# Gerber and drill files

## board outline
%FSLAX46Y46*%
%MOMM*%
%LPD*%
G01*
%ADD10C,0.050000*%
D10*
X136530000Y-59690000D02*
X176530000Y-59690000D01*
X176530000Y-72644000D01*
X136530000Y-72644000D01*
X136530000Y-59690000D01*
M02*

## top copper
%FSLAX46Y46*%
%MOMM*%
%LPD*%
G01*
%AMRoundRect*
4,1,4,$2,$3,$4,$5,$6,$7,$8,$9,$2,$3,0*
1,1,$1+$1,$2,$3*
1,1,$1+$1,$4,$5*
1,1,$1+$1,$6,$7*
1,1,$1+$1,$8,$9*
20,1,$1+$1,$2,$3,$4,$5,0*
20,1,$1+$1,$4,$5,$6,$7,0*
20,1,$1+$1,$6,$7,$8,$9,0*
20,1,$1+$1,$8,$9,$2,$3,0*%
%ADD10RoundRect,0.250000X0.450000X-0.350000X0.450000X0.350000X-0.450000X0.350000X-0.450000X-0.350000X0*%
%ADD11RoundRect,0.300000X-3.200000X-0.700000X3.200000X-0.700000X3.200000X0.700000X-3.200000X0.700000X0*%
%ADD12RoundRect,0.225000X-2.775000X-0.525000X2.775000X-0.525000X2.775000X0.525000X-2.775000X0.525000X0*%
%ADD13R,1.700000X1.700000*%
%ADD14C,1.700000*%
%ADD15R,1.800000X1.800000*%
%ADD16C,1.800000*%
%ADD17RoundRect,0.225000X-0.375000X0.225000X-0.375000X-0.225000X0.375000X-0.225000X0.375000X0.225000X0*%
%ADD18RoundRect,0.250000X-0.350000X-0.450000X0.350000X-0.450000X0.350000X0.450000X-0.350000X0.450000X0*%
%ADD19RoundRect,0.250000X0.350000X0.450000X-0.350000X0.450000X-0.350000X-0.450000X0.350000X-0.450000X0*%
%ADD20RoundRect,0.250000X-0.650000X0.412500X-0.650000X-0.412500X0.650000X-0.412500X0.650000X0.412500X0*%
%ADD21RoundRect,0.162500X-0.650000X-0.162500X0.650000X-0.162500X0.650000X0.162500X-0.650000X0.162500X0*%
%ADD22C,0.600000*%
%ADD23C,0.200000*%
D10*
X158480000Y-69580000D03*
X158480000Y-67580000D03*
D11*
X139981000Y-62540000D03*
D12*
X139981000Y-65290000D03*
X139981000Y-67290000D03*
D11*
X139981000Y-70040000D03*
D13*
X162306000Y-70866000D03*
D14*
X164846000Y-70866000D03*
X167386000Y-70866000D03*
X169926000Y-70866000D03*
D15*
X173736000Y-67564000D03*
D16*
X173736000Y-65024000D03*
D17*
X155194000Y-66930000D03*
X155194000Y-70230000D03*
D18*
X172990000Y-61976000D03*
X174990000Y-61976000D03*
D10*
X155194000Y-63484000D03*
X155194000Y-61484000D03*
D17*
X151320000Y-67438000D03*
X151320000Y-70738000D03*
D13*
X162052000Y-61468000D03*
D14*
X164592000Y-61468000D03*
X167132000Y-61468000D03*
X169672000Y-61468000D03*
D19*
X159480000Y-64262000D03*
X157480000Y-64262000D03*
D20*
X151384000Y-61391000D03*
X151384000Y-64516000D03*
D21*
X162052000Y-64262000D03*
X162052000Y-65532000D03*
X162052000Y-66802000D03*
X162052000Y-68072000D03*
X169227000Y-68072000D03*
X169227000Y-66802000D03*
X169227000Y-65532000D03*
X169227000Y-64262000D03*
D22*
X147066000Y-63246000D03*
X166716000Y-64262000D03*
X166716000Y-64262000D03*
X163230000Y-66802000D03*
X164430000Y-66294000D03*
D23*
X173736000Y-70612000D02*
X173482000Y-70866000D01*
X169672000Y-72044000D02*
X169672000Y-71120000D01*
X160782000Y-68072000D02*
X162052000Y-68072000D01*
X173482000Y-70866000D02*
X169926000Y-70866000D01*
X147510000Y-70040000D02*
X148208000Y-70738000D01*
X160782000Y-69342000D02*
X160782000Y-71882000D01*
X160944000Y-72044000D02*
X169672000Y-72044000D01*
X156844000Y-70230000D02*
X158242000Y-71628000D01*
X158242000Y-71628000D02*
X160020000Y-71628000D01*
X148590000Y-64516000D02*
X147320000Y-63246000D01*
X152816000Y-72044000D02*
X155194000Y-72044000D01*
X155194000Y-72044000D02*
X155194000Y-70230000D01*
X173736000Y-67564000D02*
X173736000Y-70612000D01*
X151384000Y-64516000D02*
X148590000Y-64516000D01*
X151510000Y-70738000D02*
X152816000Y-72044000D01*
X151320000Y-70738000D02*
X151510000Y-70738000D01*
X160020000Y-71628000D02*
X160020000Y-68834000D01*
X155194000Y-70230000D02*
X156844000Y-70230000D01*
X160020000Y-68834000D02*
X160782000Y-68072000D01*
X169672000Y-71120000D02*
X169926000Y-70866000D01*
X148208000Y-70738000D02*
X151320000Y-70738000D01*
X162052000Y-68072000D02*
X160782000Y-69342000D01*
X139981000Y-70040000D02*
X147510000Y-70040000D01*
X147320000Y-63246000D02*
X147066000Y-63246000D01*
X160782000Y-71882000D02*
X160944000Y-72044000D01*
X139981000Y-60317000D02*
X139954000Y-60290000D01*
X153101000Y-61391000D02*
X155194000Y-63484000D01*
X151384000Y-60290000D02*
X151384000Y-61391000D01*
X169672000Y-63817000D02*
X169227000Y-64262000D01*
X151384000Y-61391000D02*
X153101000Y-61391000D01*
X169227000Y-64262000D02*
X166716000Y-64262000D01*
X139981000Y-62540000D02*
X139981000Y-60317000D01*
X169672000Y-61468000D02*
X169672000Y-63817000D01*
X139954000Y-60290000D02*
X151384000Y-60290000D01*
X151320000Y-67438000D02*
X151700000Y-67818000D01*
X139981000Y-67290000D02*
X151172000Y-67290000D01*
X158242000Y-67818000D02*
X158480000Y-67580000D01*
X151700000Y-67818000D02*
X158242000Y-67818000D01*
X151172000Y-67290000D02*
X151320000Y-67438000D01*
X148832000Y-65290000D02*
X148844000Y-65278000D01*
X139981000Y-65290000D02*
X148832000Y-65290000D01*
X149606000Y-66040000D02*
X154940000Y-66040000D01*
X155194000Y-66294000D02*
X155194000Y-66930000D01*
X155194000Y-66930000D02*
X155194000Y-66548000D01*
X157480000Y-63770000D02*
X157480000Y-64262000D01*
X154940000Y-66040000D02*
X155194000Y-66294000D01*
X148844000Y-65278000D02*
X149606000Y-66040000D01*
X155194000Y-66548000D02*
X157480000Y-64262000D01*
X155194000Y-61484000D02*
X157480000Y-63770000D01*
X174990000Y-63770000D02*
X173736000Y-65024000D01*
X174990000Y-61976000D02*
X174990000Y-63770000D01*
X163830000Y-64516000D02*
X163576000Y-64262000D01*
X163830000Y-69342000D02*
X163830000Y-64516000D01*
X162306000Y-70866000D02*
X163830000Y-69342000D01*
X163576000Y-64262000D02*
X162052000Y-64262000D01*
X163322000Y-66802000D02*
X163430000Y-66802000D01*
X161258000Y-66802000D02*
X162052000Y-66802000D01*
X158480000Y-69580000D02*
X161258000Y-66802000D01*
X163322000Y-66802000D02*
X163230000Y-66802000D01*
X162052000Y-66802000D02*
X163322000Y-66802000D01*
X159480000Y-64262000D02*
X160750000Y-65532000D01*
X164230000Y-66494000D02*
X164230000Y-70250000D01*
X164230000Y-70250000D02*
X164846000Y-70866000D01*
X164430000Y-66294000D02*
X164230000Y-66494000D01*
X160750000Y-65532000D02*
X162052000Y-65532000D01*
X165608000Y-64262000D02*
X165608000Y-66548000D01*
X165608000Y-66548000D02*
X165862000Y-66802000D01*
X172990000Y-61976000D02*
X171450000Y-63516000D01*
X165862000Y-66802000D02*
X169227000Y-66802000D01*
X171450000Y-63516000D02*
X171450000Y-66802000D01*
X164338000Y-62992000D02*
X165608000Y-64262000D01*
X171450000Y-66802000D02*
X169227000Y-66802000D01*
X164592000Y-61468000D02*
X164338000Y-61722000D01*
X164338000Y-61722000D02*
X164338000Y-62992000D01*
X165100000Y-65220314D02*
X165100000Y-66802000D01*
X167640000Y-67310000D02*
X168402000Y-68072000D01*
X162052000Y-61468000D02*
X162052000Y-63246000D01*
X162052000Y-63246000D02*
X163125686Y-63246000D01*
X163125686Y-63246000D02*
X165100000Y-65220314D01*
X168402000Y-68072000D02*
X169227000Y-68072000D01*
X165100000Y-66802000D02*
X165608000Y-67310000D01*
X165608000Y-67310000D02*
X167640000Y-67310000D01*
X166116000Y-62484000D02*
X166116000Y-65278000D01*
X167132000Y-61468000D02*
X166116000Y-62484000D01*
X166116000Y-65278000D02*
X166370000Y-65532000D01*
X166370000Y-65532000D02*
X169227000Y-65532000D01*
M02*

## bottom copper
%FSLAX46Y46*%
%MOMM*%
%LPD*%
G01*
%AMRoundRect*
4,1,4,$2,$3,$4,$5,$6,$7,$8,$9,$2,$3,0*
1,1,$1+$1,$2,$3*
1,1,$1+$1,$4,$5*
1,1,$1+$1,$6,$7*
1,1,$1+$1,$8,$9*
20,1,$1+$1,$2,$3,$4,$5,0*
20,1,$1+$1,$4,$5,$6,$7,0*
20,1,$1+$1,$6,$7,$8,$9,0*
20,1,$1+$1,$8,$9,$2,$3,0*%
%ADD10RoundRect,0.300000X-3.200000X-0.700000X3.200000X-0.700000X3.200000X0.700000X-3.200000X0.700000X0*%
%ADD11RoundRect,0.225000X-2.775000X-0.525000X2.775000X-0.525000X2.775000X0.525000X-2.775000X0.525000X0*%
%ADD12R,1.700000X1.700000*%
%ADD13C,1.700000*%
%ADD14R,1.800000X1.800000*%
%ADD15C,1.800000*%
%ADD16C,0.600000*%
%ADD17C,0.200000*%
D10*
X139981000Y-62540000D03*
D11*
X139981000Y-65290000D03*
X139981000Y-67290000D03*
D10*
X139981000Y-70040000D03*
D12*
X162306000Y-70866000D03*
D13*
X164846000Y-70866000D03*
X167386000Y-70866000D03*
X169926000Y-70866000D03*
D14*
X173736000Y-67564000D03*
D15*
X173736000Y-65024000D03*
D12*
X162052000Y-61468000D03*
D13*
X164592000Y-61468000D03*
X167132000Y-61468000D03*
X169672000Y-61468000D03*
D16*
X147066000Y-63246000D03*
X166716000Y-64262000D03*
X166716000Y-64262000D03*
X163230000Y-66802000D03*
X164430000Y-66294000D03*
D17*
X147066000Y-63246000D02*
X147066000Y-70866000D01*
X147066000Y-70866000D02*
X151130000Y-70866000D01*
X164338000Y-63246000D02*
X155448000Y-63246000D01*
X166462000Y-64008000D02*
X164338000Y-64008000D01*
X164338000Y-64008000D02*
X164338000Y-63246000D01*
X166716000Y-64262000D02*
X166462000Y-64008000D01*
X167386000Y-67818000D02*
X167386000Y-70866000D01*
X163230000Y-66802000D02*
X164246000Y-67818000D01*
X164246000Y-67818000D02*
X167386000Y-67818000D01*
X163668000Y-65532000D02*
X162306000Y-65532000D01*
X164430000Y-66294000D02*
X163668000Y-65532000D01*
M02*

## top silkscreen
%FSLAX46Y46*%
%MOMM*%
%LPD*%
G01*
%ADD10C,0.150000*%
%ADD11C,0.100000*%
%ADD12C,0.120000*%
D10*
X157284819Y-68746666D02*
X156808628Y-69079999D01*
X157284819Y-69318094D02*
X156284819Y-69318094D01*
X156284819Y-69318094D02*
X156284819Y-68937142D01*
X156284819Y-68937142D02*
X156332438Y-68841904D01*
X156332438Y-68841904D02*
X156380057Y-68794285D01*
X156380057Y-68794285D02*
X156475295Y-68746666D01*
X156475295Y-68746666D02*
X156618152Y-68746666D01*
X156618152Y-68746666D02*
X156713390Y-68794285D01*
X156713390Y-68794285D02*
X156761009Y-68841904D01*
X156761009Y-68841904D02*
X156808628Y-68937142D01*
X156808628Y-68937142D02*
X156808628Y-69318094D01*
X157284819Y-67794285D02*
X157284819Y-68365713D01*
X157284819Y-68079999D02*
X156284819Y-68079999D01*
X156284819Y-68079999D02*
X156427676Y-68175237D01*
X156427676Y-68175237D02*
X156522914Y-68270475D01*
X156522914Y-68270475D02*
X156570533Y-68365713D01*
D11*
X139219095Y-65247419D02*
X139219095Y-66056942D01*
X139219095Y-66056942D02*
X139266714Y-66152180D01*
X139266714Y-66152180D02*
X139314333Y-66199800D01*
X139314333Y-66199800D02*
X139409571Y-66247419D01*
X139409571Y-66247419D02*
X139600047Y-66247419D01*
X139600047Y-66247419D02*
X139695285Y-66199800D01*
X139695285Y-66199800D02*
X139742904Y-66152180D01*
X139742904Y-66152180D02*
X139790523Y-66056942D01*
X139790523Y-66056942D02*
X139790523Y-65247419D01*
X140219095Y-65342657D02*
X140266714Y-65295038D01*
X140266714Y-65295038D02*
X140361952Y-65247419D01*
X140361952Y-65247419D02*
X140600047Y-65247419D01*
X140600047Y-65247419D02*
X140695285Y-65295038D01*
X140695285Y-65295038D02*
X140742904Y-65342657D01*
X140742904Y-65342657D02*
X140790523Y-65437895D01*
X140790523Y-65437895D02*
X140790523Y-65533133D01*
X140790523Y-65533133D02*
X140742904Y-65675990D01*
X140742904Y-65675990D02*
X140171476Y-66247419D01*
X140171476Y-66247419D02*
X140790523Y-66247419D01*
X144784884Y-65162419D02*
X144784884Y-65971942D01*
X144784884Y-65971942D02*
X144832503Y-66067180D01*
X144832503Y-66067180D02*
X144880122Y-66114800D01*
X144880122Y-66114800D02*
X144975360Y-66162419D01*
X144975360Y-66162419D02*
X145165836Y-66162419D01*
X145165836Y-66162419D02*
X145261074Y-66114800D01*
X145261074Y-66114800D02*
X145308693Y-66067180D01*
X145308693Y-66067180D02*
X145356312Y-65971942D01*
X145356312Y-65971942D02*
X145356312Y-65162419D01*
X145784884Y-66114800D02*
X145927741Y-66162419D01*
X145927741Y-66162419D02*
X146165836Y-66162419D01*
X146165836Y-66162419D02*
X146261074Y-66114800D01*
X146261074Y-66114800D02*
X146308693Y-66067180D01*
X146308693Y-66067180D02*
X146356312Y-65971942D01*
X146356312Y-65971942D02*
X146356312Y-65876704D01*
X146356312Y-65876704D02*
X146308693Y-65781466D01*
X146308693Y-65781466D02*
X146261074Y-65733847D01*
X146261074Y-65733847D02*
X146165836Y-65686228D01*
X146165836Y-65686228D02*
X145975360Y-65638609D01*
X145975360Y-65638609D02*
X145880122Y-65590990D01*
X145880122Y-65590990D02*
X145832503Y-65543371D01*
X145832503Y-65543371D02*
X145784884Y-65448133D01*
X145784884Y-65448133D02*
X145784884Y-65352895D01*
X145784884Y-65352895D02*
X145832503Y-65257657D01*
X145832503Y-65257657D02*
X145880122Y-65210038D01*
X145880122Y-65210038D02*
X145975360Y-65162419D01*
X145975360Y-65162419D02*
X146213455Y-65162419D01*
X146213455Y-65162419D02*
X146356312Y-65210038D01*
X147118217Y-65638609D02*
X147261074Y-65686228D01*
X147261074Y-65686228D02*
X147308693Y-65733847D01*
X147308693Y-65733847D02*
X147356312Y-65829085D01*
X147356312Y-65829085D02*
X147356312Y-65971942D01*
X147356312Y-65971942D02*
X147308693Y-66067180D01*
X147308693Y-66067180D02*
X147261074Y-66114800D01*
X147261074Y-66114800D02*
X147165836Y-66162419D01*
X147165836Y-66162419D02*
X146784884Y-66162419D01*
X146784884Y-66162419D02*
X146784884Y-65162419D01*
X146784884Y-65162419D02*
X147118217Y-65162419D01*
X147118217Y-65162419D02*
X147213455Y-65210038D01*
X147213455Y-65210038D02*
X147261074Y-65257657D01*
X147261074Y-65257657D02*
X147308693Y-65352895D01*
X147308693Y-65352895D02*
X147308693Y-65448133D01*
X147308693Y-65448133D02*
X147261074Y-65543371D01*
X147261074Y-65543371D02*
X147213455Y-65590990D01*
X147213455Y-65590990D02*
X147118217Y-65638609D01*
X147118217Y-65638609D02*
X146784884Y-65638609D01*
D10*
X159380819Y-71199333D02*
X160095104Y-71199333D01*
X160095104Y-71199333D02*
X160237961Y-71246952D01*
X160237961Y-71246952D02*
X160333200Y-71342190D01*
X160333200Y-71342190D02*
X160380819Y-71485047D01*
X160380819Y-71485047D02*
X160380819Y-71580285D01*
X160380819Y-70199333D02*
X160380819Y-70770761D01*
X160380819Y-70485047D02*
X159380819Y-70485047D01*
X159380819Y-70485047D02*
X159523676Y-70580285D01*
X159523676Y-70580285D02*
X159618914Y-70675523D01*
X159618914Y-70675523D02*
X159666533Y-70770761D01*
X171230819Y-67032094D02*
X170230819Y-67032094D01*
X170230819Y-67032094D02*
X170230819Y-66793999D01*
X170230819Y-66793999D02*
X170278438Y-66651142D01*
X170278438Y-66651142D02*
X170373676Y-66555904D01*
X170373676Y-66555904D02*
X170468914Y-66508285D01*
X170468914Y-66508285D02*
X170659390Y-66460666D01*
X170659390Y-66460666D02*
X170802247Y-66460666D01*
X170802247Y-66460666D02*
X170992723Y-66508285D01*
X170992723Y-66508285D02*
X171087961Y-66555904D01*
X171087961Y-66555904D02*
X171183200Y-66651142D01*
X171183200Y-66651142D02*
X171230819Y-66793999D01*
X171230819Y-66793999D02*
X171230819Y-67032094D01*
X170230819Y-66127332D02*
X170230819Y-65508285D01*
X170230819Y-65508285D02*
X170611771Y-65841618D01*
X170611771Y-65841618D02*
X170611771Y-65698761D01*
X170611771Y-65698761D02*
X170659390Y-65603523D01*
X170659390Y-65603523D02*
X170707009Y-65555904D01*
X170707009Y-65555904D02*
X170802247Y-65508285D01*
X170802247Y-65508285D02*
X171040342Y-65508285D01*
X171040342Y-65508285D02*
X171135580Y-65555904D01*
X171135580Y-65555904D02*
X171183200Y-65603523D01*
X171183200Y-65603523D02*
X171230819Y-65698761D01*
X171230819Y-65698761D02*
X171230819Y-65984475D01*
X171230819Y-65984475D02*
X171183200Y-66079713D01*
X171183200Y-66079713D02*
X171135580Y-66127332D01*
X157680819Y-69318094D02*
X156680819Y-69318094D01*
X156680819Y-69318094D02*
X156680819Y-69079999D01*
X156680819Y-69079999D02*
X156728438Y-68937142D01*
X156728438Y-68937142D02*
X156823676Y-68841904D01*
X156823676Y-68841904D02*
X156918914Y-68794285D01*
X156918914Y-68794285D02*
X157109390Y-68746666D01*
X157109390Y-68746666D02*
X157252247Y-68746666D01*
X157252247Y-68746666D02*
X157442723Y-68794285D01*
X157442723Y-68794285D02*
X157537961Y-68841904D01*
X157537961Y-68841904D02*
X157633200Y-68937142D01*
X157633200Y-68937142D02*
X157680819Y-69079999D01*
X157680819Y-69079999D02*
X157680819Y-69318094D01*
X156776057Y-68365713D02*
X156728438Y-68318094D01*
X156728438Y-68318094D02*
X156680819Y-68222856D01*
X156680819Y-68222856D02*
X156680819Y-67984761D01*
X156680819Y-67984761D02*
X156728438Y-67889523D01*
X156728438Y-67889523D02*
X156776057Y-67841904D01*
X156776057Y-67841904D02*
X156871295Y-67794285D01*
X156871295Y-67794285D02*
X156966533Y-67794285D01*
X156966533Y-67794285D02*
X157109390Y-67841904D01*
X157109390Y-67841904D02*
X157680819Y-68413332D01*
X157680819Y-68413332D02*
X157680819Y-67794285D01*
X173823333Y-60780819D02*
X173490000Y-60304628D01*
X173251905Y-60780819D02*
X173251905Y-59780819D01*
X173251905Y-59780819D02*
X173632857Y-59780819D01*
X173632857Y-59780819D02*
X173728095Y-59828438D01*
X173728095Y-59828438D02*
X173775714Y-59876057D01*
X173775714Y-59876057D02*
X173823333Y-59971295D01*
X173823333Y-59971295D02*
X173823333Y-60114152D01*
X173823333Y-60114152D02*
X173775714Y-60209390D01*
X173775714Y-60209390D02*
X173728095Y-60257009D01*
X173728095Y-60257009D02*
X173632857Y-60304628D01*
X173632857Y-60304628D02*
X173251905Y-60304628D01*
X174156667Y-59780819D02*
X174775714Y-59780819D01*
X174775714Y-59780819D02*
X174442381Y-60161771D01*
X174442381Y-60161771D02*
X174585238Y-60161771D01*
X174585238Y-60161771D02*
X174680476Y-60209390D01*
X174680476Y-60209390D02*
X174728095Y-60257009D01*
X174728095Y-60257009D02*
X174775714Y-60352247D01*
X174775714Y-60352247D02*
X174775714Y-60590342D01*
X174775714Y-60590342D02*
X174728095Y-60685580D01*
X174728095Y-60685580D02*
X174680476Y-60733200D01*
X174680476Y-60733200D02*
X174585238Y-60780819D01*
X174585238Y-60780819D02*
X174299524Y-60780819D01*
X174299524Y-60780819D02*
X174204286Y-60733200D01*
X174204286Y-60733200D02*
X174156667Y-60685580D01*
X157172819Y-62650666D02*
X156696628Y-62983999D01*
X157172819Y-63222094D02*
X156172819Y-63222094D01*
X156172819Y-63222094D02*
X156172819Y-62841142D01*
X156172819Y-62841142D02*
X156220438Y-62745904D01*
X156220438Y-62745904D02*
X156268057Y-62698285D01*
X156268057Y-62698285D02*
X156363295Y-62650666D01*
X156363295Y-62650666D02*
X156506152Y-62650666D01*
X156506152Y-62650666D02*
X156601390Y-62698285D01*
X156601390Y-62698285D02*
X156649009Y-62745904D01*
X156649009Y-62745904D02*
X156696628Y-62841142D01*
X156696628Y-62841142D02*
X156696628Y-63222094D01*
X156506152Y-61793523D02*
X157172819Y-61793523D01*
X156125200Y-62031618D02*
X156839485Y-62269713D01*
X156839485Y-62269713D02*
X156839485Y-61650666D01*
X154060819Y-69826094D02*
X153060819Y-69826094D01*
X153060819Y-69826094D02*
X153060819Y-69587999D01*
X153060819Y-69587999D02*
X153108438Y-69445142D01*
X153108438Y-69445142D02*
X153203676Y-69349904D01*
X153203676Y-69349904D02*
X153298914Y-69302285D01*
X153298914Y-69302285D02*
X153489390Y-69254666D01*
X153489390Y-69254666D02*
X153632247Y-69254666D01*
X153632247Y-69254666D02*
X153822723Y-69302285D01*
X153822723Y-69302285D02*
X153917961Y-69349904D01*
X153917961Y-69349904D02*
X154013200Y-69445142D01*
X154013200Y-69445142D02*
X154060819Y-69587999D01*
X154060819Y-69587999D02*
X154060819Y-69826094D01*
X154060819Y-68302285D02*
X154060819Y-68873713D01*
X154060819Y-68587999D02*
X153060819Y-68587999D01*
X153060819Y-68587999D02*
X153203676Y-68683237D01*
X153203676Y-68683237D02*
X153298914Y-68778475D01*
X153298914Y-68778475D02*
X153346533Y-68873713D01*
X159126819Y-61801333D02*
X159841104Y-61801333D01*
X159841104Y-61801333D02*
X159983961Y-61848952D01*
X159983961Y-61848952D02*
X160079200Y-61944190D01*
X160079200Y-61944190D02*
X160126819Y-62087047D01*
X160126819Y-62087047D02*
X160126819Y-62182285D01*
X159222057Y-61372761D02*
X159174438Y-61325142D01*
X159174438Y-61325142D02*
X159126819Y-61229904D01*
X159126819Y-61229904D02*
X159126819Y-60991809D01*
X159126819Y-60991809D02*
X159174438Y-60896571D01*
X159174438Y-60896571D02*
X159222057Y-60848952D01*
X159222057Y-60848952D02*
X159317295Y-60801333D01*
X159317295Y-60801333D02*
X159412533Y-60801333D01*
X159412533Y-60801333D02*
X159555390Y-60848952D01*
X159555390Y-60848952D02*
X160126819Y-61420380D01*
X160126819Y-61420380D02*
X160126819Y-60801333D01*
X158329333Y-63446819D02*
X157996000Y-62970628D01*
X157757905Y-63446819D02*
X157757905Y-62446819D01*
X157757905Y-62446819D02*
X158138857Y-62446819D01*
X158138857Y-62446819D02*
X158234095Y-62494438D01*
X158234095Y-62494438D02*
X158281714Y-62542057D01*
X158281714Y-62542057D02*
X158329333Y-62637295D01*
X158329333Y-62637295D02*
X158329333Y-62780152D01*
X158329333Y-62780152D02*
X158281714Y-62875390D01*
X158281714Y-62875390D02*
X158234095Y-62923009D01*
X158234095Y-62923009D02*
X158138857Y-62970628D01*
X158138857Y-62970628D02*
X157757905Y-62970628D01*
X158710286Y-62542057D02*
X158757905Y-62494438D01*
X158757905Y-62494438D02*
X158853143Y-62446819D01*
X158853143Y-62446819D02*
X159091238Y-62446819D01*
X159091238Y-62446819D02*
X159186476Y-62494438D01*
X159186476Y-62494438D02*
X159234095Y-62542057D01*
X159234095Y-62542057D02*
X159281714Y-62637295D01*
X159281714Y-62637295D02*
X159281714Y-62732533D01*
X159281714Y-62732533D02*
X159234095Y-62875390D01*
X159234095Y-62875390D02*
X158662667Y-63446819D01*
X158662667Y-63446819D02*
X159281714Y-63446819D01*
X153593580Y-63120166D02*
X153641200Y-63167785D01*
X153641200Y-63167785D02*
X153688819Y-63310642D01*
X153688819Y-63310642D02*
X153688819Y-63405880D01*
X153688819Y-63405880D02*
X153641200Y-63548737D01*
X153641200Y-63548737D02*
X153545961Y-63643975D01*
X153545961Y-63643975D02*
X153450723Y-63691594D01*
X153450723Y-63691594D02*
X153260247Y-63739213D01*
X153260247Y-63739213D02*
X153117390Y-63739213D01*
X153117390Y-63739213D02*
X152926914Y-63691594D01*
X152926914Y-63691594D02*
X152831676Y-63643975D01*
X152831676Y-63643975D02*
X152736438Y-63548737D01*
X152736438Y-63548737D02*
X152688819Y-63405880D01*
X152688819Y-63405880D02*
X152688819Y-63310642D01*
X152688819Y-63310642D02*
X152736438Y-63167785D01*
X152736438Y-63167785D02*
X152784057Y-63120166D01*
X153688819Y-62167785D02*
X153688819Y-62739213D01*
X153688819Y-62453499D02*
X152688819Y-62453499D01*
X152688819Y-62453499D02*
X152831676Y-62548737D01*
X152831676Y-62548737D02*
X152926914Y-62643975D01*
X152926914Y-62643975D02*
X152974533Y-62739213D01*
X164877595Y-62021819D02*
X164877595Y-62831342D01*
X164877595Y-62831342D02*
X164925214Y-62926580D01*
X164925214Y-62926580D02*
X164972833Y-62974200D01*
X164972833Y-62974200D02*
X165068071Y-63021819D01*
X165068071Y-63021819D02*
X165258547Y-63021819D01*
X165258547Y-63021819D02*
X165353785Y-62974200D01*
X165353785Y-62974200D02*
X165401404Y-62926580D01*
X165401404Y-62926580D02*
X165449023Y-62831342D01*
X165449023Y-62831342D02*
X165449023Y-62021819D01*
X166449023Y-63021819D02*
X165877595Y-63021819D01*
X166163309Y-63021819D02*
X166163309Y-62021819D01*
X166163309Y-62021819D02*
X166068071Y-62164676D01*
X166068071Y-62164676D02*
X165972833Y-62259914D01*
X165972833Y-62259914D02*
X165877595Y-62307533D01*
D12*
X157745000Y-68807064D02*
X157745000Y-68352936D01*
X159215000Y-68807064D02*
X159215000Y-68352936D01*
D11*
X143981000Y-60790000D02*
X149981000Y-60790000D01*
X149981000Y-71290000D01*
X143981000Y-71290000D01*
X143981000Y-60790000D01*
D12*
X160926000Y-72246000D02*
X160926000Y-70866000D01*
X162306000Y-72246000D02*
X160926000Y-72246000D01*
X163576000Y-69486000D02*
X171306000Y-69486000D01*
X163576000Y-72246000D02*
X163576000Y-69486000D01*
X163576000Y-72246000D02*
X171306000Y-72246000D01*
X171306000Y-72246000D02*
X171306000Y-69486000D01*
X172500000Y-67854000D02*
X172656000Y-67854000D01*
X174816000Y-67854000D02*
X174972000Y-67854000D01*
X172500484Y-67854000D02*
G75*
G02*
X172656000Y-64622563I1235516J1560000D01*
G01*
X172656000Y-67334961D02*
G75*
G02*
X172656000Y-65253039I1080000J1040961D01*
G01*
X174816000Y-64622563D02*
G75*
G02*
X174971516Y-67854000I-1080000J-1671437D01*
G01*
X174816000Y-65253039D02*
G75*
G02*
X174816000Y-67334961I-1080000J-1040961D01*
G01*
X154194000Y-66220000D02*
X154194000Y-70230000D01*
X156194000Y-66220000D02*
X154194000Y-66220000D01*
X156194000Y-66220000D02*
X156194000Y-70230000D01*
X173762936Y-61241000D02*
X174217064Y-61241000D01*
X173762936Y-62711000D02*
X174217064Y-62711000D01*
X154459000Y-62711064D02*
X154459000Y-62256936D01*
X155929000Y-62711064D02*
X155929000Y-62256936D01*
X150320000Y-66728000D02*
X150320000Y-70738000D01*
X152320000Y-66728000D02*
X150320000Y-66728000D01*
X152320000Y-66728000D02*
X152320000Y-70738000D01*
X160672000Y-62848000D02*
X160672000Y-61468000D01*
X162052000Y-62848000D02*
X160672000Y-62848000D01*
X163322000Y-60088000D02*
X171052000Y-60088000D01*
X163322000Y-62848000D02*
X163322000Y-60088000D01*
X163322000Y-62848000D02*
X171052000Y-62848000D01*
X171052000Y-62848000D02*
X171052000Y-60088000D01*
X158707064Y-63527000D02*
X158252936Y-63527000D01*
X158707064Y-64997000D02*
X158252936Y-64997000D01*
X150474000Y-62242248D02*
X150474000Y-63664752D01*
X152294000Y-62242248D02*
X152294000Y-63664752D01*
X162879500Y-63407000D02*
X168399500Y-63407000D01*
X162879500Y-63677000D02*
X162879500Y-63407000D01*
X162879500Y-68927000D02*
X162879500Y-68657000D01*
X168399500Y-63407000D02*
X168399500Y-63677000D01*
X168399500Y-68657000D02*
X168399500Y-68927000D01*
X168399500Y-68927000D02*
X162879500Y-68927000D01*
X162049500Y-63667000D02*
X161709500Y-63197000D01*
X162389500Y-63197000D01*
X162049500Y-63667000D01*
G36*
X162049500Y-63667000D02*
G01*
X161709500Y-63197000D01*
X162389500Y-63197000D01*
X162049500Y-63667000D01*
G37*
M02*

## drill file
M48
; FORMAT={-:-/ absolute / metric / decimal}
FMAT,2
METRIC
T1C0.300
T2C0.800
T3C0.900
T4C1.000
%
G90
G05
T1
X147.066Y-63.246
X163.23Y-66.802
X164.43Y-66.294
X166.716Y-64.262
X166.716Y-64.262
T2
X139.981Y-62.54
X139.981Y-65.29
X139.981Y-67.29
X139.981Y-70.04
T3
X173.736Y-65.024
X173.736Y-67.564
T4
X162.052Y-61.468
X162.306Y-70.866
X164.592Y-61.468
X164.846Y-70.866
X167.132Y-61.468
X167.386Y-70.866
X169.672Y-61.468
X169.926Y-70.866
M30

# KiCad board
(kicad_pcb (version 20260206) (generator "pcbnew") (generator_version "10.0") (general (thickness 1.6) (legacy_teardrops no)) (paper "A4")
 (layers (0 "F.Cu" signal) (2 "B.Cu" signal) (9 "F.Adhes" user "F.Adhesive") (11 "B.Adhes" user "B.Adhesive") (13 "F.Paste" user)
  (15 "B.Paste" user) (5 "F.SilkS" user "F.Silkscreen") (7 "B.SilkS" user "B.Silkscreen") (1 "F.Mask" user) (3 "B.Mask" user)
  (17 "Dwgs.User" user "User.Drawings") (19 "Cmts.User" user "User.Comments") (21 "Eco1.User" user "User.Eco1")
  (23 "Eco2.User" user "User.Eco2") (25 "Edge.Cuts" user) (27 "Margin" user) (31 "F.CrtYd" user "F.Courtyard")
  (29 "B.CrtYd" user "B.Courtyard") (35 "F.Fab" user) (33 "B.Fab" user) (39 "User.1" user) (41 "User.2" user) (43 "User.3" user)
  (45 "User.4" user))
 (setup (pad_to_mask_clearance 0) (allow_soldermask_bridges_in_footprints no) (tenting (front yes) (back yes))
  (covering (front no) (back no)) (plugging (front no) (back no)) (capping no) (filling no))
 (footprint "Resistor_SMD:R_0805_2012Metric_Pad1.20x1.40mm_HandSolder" (layer "F.Cu") (at 158.48 68.58 90)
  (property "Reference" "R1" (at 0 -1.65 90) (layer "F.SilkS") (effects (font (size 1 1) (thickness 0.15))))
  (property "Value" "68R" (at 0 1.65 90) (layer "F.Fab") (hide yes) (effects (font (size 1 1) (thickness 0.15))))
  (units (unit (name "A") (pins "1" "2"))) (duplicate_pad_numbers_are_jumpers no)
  (fp_line (start -0.227064 -0.735) (end 0.227064 -0.735) (stroke (width 0.12) (type solid)) (layer "F.SilkS"))
  (fp_line (start -0.227064 0.735) (end 0.227064 0.735) (stroke (width 0.12) (type solid)) (layer "F.SilkS"))
  (pad "1" smd roundrect (at -1 0 90) (size 1.2 1.4) (layers "F.Cu" "F.Mask" "F.Paste") (roundrect_rratio 0.208333) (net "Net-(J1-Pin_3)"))
  (pad "2" smd roundrect (at 1 0 90) (size 1.2 1.4) (layers "F.Cu" "F.Mask" "F.Paste") (roundrect_rratio 0.208333) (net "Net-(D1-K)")))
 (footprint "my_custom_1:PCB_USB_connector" (layer "F.Cu") (at 139.981 66.29)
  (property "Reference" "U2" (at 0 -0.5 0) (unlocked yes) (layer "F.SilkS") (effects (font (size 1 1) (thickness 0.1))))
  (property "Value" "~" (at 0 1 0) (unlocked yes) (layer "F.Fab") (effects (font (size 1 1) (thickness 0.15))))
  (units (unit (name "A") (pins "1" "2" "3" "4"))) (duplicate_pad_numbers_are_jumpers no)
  (fp_rect (start 4 -5.5) (end 10 5) (stroke (width 0.1) (type default)) (fill no) (layer "F.SilkS"))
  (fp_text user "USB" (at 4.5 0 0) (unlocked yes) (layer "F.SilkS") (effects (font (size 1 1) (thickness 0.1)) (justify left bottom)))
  (pad "1" thru_hole roundrect (at 0 -3.75) (size 7 2) (drill 0.8) (layers "*.Cu" "*.Mask") (remove_unused_layers no)
   (roundrect_rratio 0.15) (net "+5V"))
  (pad "2" thru_hole roundrect (at 0 -1) (size 6 1.5) (drill 0.8) (layers "*.Cu" "*.Mask") (remove_unused_layers no) (roundrect_rratio 0.15)
   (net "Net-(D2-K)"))
  (pad "3" thru_hole roundrect (at 0 1) (size 6 1.5) (drill 0.8) (layers "*.Cu" "*.Mask") (remove_unused_layers no) (roundrect_rratio 0.15)
   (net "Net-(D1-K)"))
  (pad "4" thru_hole roundrect (at 0 3.75) (size 7 2) (drill 0.8) (layers "*.Cu" "*.Mask") (remove_unused_layers no) (roundrect_rratio 0.15)
   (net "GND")))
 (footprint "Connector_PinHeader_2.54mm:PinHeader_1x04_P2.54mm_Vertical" (layer "F.Cu") (at 162.306 70.866 90)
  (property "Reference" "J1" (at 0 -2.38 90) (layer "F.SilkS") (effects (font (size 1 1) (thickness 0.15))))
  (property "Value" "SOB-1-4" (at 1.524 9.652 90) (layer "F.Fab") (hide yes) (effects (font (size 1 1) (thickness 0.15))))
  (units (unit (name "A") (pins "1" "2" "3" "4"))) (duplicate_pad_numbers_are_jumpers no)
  (fp_line (start -1.38 -1.38) (end 0 -1.38) (stroke (width 0.12) (type solid)) (layer "F.SilkS"))
  (fp_line (start -1.38 0) (end -1.38 -1.38) (stroke (width 0.12) (type solid)) (layer "F.SilkS"))
  (fp_line (start 1.38 1.27) (end 1.38 9) (stroke (width 0.12) (type solid)) (layer "F.SilkS"))
  (fp_line (start -1.38 1.27) (end 1.38 1.27) (stroke (width 0.12) (type solid)) (layer "F.SilkS"))
  (fp_line (start -1.38 1.27) (end -1.38 9) (stroke (width 0.12) (type solid)) (layer "F.SilkS"))
  (fp_line (start -1.38 9) (end 1.38 9) (stroke (width 0.12) (type solid)) (layer "F.SilkS"))
  (pad "1" thru_hole rect (at 0 0 90) (size 1.7 1.7) (drill 1) (layers "*.Cu" "*.Mask") (remove_unused_layers no) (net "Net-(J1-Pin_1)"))
  (pad "2" thru_hole circle (at 0 2.54 90) (size 1.7 1.7) (drill 1) (layers "*.Cu" "*.Mask") (remove_unused_layers no)
   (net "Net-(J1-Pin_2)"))
  (pad "3" thru_hole circle (at 0 5.08 90) (size 1.7 1.7) (drill 1) (layers "*.Cu" "*.Mask") (remove_unused_layers no)
   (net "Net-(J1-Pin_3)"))
  (pad "4" thru_hole circle (at 0 7.62 90) (size 1.7 1.7) (drill 1) (layers "*.Cu" "*.Mask") (remove_unused_layers no) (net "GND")))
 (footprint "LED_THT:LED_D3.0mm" (layer "F.Cu") (at 173.736 67.564 90)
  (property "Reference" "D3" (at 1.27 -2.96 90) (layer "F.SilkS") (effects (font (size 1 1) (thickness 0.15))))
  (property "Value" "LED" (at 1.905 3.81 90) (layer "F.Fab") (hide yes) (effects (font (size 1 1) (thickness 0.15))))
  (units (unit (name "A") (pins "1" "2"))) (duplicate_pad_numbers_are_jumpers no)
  (fp_line (start -0.29 -1.236) (end -0.29 -1.08) (stroke (width 0.12) (type solid)) (layer "F.SilkS"))
  (fp_line (start -0.29 1.08) (end -0.29 1.236) (stroke (width 0.12) (type solid)) (layer "F.SilkS"))
  (fp_arc (start -0.29 -1.235516) (mid 1.36566 -1.987699) (end 2.941437 -1.08) (stroke (width 0.12) (type solid)) (layer "F.SilkS"))
  (fp_arc (start 0.229039 -1.08) (mid 1.27 -1.5) (end 2.310961 -1.08) (stroke (width 0.12) (type solid)) (layer "F.SilkS"))
  (fp_arc (start 2.941437 1.08) (mid 1.36566 1.987699) (end -0.29 1.235516) (stroke (width 0.12) (type solid)) (layer "F.SilkS"))
  (fp_arc (start 2.310961 1.08) (mid 1.27 1.5) (end 0.229039 1.08) (stroke (width 0.12) (type solid)) (layer "F.SilkS"))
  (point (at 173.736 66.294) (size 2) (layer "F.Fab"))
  (pad "1" thru_hole rect (at 0 0 90) (size 1.8 1.8) (drill 0.9) (layers "*.Cu" "*.Mask") (remove_unused_layers no) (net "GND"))
  (pad "2" thru_hole circle (at 2.54 0 90) (size 1.8 1.8) (drill 0.9) (layers "*.Cu" "*.Mask") (remove_unused_layers no) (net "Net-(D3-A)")))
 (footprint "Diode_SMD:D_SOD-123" (layer "F.Cu") (at 155.194 68.58 -90)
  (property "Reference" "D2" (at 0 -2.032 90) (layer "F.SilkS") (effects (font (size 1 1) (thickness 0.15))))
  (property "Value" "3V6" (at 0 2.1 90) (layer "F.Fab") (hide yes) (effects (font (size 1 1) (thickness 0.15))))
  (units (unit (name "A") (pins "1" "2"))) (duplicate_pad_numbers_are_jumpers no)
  (fp_line (start -2.36 1) (end 1.65 1) (stroke (width 0.12) (type solid)) (layer "F.SilkS"))
  (fp_line (start -2.36 -1) (end -2.36 1) (stroke (width 0.12) (type solid)) (layer "F.SilkS"))
  (fp_line (start -2.36 -1) (end 1.65 -1) (stroke (width 0.12) (type solid)) (layer "F.SilkS"))
  (pad "1" smd roundrect (at -1.65 0 270) (size 0.9 1.2) (layers "F.Cu" "F.Mask" "F.Paste") (roundrect_rratio 0.25) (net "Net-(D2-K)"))
  (pad "2" smd roundrect (at 1.65 0 270) (size 0.9 1.2) (layers "F.Cu" "F.Mask" "F.Paste") (roundrect_rratio 0.25) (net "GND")))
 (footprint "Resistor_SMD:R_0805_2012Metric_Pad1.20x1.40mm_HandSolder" (layer "F.Cu") (at 173.99 61.976)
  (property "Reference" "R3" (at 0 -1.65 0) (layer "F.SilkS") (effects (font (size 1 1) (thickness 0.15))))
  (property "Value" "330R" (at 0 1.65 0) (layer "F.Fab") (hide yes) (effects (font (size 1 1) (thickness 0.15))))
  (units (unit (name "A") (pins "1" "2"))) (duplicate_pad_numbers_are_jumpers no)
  (fp_line (start -0.227064 -0.735) (end 0.227064 -0.735) (stroke (width 0.12) (type solid)) (layer "F.SilkS"))
  (fp_line (start -0.227064 0.735) (end 0.227064 0.735) (stroke (width 0.12) (type solid)) (layer "F.SilkS"))
  (pad "1" smd roundrect (at -1 0) (size 1.2 1.4) (layers "F.Cu" "F.Mask" "F.Paste") (roundrect_rratio 0.208333) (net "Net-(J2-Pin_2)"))
  (pad "2" smd roundrect (at 1 0) (size 1.2 1.4) (layers "F.Cu" "F.Mask" "F.Paste") (roundrect_rratio 0.208333) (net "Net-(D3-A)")))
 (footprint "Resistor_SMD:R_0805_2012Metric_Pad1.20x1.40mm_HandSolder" (layer "F.Cu") (at 155.194 62.484 90)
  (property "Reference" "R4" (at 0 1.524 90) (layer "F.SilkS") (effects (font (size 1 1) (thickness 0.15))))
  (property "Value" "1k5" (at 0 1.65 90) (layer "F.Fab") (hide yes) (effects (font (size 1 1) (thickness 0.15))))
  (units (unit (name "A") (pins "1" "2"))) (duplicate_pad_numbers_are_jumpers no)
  (fp_line (start -0.227064 -0.735) (end 0.227064 -0.735) (stroke (width 0.12) (type solid)) (layer "F.SilkS"))
  (fp_line (start -0.227064 0.735) (end 0.227064 0.735) (stroke (width 0.12) (type solid)) (layer "F.SilkS"))
  (pad "1" smd roundrect (at -1 0 90) (size 1.2 1.4) (layers "F.Cu" "F.Mask" "F.Paste") (roundrect_rratio 0.208333) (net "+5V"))
  (pad "2" smd roundrect (at 1 0 90) (size 1.2 1.4) (layers "F.Cu" "F.Mask" "F.Paste") (roundrect_rratio 0.208333) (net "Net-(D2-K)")))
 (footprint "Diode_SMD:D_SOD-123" (layer "F.Cu") (at 151.32 69.088 -90)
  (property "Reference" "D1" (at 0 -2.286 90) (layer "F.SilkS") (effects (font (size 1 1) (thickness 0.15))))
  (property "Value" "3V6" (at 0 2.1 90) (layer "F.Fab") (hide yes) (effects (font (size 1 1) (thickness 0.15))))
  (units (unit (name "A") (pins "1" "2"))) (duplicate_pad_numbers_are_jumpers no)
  (fp_line (start -2.36 1) (end 1.65 1) (stroke (width 0.12) (type solid)) (layer "F.SilkS"))
  (fp_line (start -2.36 -1) (end -2.36 1) (stroke (width 0.12) (type solid)) (layer "F.SilkS"))
  (fp_line (start -2.36 -1) (end 1.65 -1) (stroke (width 0.12) (type solid)) (layer "F.SilkS"))
  (pad "1" smd roundrect (at -1.65 0 270) (size 0.9 1.2) (layers "F.Cu" "F.Mask" "F.Paste") (roundrect_rratio 0.25) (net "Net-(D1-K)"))
  (pad "2" smd roundrect (at 1.65 0 270) (size 0.9 1.2) (layers "F.Cu" "F.Mask" "F.Paste") (roundrect_rratio 0.25) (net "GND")))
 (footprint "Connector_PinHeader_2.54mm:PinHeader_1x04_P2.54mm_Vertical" (layer "F.Cu") (at 162.052 61.468 90)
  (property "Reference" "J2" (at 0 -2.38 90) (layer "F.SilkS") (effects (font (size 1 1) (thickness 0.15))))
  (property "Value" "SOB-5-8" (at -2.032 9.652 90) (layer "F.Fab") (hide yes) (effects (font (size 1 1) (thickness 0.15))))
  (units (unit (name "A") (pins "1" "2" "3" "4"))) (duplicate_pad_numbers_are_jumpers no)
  (fp_line (start -1.38 -1.38) (end 0 -1.38) (stroke (width 0.12) (type solid)) (layer "F.SilkS"))
  (fp_line (start -1.38 0) (end -1.38 -1.38) (stroke (width 0.12) (type solid)) (layer "F.SilkS"))
  (fp_line (start 1.38 1.27) (end 1.38 9) (stroke (width 0.12) (type solid)) (layer "F.SilkS"))
  (fp_line (start -1.38 1.27) (end 1.38 1.27) (stroke (width 0.12) (type solid)) (layer "F.SilkS"))
  (fp_line (start -1.38 1.27) (end -1.38 9) (stroke (width 0.12) (type solid)) (layer "F.SilkS"))
  (fp_line (start -1.38 9) (end 1.38 9) (stroke (width 0.12) (type solid)) (layer "F.SilkS"))
  (pad "1" thru_hole rect (at 0 0 90) (size 1.7 1.7) (drill 1) (layers "*.Cu" "*.Mask") (remove_unused_layers no) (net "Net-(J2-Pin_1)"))
  (pad "2" thru_hole circle (at 0 2.54 90) (size 1.7 1.7) (drill 1) (layers "*.Cu" "*.Mask") (remove_unused_layers no)
   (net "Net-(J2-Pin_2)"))
  (pad "3" thru_hole circle (at 0 5.08 90) (size 1.7 1.7) (drill 1) (layers "*.Cu" "*.Mask") (remove_unused_layers no)
   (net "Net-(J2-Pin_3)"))
  (pad "4" thru_hole circle (at 0 7.62 90) (size 1.7 1.7) (drill 1) (layers "*.Cu" "*.Mask") (remove_unused_layers no) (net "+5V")))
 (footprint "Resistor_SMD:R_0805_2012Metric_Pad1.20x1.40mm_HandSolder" (layer "F.Cu") (at 158.48 64.262 180)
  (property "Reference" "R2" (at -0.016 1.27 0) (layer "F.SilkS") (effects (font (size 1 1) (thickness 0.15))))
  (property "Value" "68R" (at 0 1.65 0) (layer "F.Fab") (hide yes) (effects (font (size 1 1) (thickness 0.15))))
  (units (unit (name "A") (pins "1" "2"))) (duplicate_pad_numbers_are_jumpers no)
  (fp_line (start -0.227064 0.735) (end 0.227064 0.735) (stroke (width 0.12) (type solid)) (layer "F.SilkS"))
  (fp_line (start -0.227064 -0.735) (end 0.227064 -0.735) (stroke (width 0.12) (type solid)) (layer "F.SilkS"))
  (pad "1" smd roundrect (at -1 0 180) (size 1.2 1.4) (layers "F.Cu" "F.Mask" "F.Paste") (roundrect_rratio 0.208333) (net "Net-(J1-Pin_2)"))
  (pad "2" smd roundrect (at 1 0 180) (size 1.2 1.4) (layers "F.Cu" "F.Mask" "F.Paste") (roundrect_rratio 0.208333) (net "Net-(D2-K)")))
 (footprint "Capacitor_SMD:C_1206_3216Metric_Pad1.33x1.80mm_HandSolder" (layer "F.Cu") (at 151.384 62.9535 -90)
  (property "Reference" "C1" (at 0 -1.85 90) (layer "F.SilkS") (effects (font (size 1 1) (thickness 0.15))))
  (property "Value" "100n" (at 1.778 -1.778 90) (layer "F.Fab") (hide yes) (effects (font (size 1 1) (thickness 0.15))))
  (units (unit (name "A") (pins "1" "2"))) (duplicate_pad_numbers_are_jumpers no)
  (fp_line (start -0.711252 0.91) (end 0.711252 0.91) (stroke (width 0.12) (type solid)) (layer "F.SilkS"))
  (fp_line (start -0.711252 -0.91) (end 0.711252 -0.91) (stroke (width 0.12) (type solid)) (layer "F.SilkS"))
  (pad "1" smd roundrect (at -1.5625 0 270) (size 1.325 1.8) (layers "F.Cu" "F.Mask" "F.Paste") (roundrect_rratio 0.188679) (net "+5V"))
  (pad "2" smd roundrect (at 1.5625 0 270) (size 1.325 1.8) (layers "F.Cu" "F.Mask" "F.Paste") (roundrect_rratio 0.188679) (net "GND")))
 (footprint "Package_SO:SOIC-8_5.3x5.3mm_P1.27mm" (layer "F.Cu") (at 165.6395 66.167)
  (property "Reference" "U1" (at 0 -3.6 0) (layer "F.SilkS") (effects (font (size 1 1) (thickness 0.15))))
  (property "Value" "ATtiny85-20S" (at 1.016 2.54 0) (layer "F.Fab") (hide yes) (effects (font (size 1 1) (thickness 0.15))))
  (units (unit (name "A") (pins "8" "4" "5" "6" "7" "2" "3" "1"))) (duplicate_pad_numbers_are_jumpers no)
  (fp_line (start -2.76 -2.76) (end 2.76 -2.76) (stroke (width 0.12) (type solid)) (layer "F.SilkS"))
  (fp_line (start -2.76 -2.49) (end -2.76 -2.76) (stroke (width 0.12) (type solid)) (layer "F.SilkS"))
  (fp_line (start -2.76 2.76) (end -2.76 2.49) (stroke (width 0.12) (type solid)) (layer "F.SilkS"))
  (fp_line (start 2.76 -2.76) (end 2.76 -2.49) (stroke (width 0.12) (type solid)) (layer "F.SilkS"))
  (fp_line (start 2.76 2.49) (end 2.76 2.76) (stroke (width 0.12) (type solid)) (layer "F.SilkS"))
  (fp_line (start 2.76 2.76) (end -2.76 2.76) (stroke (width 0.12) (type solid)) (layer "F.SilkS"))
  (fp_poly (pts (xy -3.59 -2.5) (xy -3.93 -2.97) (xy -3.25 -2.97)) (stroke (width 0.12) (type solid)) (fill yes) (layer "F.SilkS"))
  (pad "1" smd roundrect (at -3.5875 -1.905) (size 1.625 0.65) (layers "F.Cu" "F.Mask" "F.Paste") (roundrect_rratio 0.25)
   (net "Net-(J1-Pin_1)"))
  (pad "2" smd roundrect (at -3.5875 -0.635) (size 1.625 0.65) (layers "F.Cu" "F.Mask" "F.Paste") (roundrect_rratio 0.25)
   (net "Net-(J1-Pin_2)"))
  (pad "3" smd roundrect (at -3.5875 0.635) (size 1.625 0.65) (layers "F.Cu" "F.Mask" "F.Paste") (roundrect_rratio 0.25)
   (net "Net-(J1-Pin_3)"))
  (pad "4" smd roundrect (at -3.5875 1.905) (size 1.625 0.65) (layers "F.Cu" "F.Mask" "F.Paste") (roundrect_rratio 0.25) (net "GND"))
  (pad "5" smd roundrect (at 3.5875 1.905) (size 1.625 0.65) (layers "F.Cu" "F.Mask" "F.Paste") (roundrect_rratio 0.25)
   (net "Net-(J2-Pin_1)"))
  (pad "6" smd roundrect (at 3.5875 0.635) (size 1.625 0.65) (layers "F.Cu" "F.Mask" "F.Paste") (roundrect_rratio 0.25)
   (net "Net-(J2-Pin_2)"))
  (pad "7" smd roundrect (at 3.5875 -0.635) (size 1.625 0.65) (layers "F.Cu" "F.Mask" "F.Paste") (roundrect_rratio 0.25)
   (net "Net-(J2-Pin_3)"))
  (pad "8" smd roundrect (at 3.5875 -1.905) (size 1.625 0.65) (layers "F.Cu" "F.Mask" "F.Paste") (roundrect_rratio 0.25) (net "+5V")))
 (gr_rect (start 136.53 59.69) (end 176.53 72.644) (stroke (width 0.05) (type solid)) (fill no) (layer "Edge.Cuts"))
 (segment (start 173.736 70.612) (end 173.482 70.866) (width 0.2) (layer "F.Cu") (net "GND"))
 (segment (start 169.672 72.044) (end 169.672 71.12) (width 0.2) (layer "F.Cu") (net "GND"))
 (segment (start 160.782 68.072) (end 162.052 68.072) (width 0.2) (layer "F.Cu") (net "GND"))
 (segment (start 173.482 70.866) (end 169.926 70.866) (width 0.2) (layer "F.Cu") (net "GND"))
 (segment (start 147.51 70.04) (end 148.208 70.738) (width 0.2) (layer "F.Cu") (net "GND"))
 (segment (start 160.782 69.342) (end 160.782 71.882) (width 0.2) (layer "F.Cu") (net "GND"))
 (segment (start 160.944 72.044) (end 169.672 72.044) (width 0.2) (layer "F.Cu") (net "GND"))
 (segment (start 156.844 70.23) (end 158.242 71.628) (width 0.2) (layer "F.Cu") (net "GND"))
 (segment (start 158.242 71.628) (end 160.02 71.628) (width 0.2) (layer "F.Cu") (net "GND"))
 (segment (start 148.59 64.516) (end 147.32 63.246) (width 0.2) (layer "F.Cu") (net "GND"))
 (segment (start 152.816 72.044) (end 155.194 72.044) (width 0.2) (layer "F.Cu") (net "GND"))
 (segment (start 155.194 72.044) (end 155.194 70.23) (width 0.2) (layer "F.Cu") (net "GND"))
 (segment (start 173.736 67.564) (end 173.736 70.612) (width 0.2) (layer "F.Cu") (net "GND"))
 (segment (start 151.384 64.516) (end 148.59 64.516) (width 0.2) (layer "F.Cu") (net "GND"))
 (segment (start 151.51 70.738) (end 152.816 72.044) (width 0.2) (layer "F.Cu") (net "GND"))
 (segment (start 151.32 70.738) (end 151.51 70.738) (width 0.2) (layer "F.Cu") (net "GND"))
 (segment (start 160.02 71.628) (end 160.02 68.834) (width 0.2) (layer "F.Cu") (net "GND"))
 (segment (start 155.194 70.23) (end 156.844 70.23) (width 0.2) (layer "F.Cu") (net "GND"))
 (segment (start 160.02 68.834) (end 160.782 68.072) (width 0.2) (layer "F.Cu") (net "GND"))
 (segment (start 169.672 71.12) (end 169.926 70.866) (width 0.2) (layer "F.Cu") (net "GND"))
 (segment (start 148.208 70.738) (end 151.32 70.738) (width 0.2) (layer "F.Cu") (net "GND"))
 (segment (start 162.052 68.072) (end 160.782 69.342) (width 0.2) (layer "F.Cu") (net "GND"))
 (segment (start 139.981 70.04) (end 147.51 70.04) (width 0.2) (layer "F.Cu") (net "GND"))
 (segment (start 147.32 63.246) (end 147.066 63.246) (width 0.2) (layer "F.Cu") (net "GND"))
 (segment (start 160.782 71.882) (end 160.944 72.044) (width 0.2) (layer "F.Cu") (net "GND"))
 (via (at 147.066 63.246) (size 0.6) (drill 0.3) (layers "F.Cu" "B.Cu") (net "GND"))
 (segment (start 147.066 63.246) (end 147.066 70.866) (width 0.2) (layer "B.Cu") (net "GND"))
 (segment (start 147.066 70.866) (end 151.13 70.866) (width 0.2) (layer "B.Cu") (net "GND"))
 (segment (start 139.981 60.317) (end 139.954 60.29) (width 0.2) (layer "F.Cu") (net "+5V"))
 (segment (start 153.101 61.391) (end 155.194 63.484) (width 0.2) (layer "F.Cu") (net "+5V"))
 (segment (start 151.384 60.29) (end 151.384 61.391) (width 0.2) (layer "F.Cu") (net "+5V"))
 (segment (start 169.672 63.817) (end 169.227 64.262) (width 0.2) (layer "F.Cu") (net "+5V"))
 (segment (start 151.384 61.391) (end 153.101 61.391) (width 0.2) (layer "F.Cu") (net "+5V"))
 (segment (start 169.227 64.262) (end 166.716 64.262) (width 0.2) (layer "F.Cu") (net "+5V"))
 (segment (start 139.981 62.54) (end 139.981 60.317) (width 0.2) (layer "F.Cu") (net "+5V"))
 (segment (start 169.672 61.468) (end 169.672 63.817) (width 0.2) (layer "F.Cu") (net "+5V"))
 (segment (start 139.954 60.29) (end 151.384 60.29) (width 0.2) (layer "F.Cu") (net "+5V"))
 (via (at 166.716 64.262) (size 0.6) (drill 0.3) (layers "F.Cu" "B.Cu") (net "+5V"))
 (via (at 166.716 64.262) (size 0.6) (drill 0.3) (layers "F.Cu" "B.Cu") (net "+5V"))
 (segment (start 164.338 63.246) (end 155.448 63.246) (width 0.2) (layer "B.Cu") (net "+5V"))
 (segment (start 166.462 64.008) (end 164.338 64.008) (width 0.2) (layer "B.Cu") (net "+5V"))
 (segment (start 164.338 64.008) (end 164.338 63.246) (width 0.2) (layer "B.Cu") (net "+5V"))
 (segment (start 166.716 64.262) (end 166.462 64.008) (width 0.2) (layer "B.Cu") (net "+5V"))
 (segment (start 151.32 67.438) (end 151.7 67.818) (width 0.2) (layer "F.Cu") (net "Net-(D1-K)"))
 (segment (start 139.981 67.29) (end 151.172 67.29) (width 0.2) (layer "F.Cu") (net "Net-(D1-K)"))
 (segment (start 158.242 67.818) (end 158.48 67.58) (width 0.2) (layer "F.Cu") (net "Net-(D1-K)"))
 (segment (start 151.7 67.818) (end 158.242 67.818) (width 0.2) (layer "F.Cu") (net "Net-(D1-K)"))
 (segment (start 151.172 67.29) (end 151.32 67.438) (width 0.2) (layer "F.Cu") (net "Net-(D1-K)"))
 (segment (start 148.832 65.29) (end 148.844 65.278) (width 0.2) (layer "F.Cu") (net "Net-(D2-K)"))
 (segment (start 139.981 65.29) (end 148.832 65.29) (width 0.2) (layer "F.Cu") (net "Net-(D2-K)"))
 (segment (start 149.606 66.04) (end 154.94 66.04) (width 0.2) (layer "F.Cu") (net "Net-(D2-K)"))
 (segment (start 155.194 66.294) (end 155.194 66.93) (width 0.2) (layer "F.Cu") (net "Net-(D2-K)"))
 (segment (start 155.194 66.93) (end 155.194 66.548) (width 0.2) (layer "F.Cu") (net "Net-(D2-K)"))
 (segment (start 157.48 63.77) (end 157.48 64.262) (width 0.2) (layer "F.Cu") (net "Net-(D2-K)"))
 (segment (start 154.94 66.04) (end 155.194 66.294) (width 0.2) (layer "F.Cu") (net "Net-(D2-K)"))
 (segment (start 148.844 65.278) (end 149.606 66.04) (width 0.2) (layer "F.Cu") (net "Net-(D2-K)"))
 (segment (start 155.194 66.548) (end 157.48 64.262) (width 0.2) (layer "F.Cu") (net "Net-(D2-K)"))
 (segment (start 155.194 61.484) (end 157.48 63.77) (width 0.2) (layer "F.Cu") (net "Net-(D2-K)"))
 (segment (start 174.99 63.77) (end 173.736 65.024) (width 0.2) (layer "F.Cu") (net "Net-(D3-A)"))
 (segment (start 174.99 61.976) (end 174.99 63.77) (width 0.2) (layer "F.Cu") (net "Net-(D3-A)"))
 (segment (start 163.83 64.516) (end 163.576 64.262) (width 0.2) (layer "F.Cu") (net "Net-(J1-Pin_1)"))
 (segment (start 163.83 69.342) (end 163.83 64.516) (width 0.2) (layer "F.Cu") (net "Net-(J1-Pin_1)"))
 (segment (start 162.306 70.866) (end 163.83 69.342) (width 0.2) (layer "F.Cu") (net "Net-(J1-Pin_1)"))
 (segment (start 163.576 64.262) (end 162.052 64.262) (width 0.2) (layer "F.Cu") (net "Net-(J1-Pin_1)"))
 (segment (start 163.322 66.802) (end 163.43 66.802) (width 0.2) (layer "F.Cu") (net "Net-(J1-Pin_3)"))
 (segment (start 161.258 66.802) (end 162.052 66.802) (width 0.2) (layer "F.Cu") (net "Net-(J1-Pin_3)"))
 (segment (start 158.48 69.58) (end 161.258 66.802) (width 0.2) (layer "F.Cu") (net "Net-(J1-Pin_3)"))
 (segment (start 163.322 66.802) (end 163.23 66.802) (width 0.2) (layer "F.Cu") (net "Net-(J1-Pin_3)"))
 (segment (start 162.052 66.802) (end 163.322 66.802) (width 0.2) (layer "F.Cu") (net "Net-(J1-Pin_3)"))
 (via (at 163.23 66.802) (size 0.6) (drill 0.3) (layers "F.Cu" "B.Cu") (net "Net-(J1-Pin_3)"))
 (segment (start 167.386 67.818) (end 167.386 70.866) (width 0.2) (layer "B.Cu") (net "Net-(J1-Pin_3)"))
 (segment (start 163.23 66.802) (end 164.246 67.818) (width 0.2) (layer "B.Cu") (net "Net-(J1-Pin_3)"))
 (segment (start 164.246 67.818) (end 167.386 67.818) (width 0.2) (layer "B.Cu") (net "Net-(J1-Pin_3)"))
 (segment (start 159.48 64.262) (end 160.75 65.532) (width 0.2) (layer "F.Cu") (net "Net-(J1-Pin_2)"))
 (segment (start 164.23 66.494) (end 164.23 70.25) (width 0.2) (layer "F.Cu") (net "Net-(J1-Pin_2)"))
 (segment (start 164.23 70.25) (end 164.846 70.866) (width 0.2) (layer "F.Cu") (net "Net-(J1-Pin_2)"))
 (segment (start 164.43 66.294) (end 164.23 66.494) (width 0.2) (layer "F.Cu") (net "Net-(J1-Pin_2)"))
 (segment (start 160.75 65.532) (end 162.052 65.532) (width 0.2) (layer "F.Cu") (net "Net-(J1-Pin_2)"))
 (via (at 164.43 66.294) (size 0.6) (drill 0.3) (layers "F.Cu" "B.Cu") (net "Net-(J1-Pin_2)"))
 (segment (start 163.668 65.532) (end 162.306 65.532) (width 0.2) (layer "B.Cu") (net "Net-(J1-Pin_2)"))
 (segment (start 164.43 66.294) (end 163.668 65.532) (width 0.2) (layer "B.Cu") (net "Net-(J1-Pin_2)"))
 (segment (start 165.608 64.262) (end 165.608 66.548) (width 0.2) (layer "F.Cu") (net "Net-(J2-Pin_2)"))
 (segment (start 165.608 66.548) (end 165.862 66.802) (width 0.2) (layer "F.Cu") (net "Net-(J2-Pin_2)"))
 (segment (start 172.99 61.976) (end 171.45 63.516) (width 0.2) (layer "F.Cu") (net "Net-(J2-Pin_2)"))
 (segment (start 165.862 66.802) (end 169.227 66.802) (width 0.2) (layer "F.Cu") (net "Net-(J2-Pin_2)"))
 (segment (start 171.45 63.516) (end 171.45 66.802) (width 0.2) (layer "F.Cu") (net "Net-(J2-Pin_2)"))
 (segment (start 164.338 62.992) (end 165.608 64.262) (width 0.2) (layer "F.Cu") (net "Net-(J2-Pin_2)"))
 (segment (start 171.45 66.802) (end 169.227 66.802) (width 0.2) (layer "F.Cu") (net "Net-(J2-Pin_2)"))
 (segment (start 164.592 61.468) (end 164.338 61.722) (width 0.2) (layer "F.Cu") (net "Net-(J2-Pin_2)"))
 (segment (start 164.338 61.722) (end 164.338 62.992) (width 0.2) (layer "F.Cu") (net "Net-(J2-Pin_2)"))
 (segment (start 165.1 65.220314) (end 165.1 66.802) (width 0.2) (layer "F.Cu") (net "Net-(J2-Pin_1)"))
 (segment (start 167.64 67.31) (end 168.402 68.072) (width 0.2) (layer "F.Cu") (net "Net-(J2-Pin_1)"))
 (segment (start 162.052 61.468) (end 162.052 63.246) (width 0.2) (layer "F.Cu") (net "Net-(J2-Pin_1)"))
 (segment (start 162.052 63.246) (end 163.125686 63.246) (width 0.2) (layer "F.Cu") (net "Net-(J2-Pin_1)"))
 (segment (start 163.125686 63.246) (end 165.1 65.220314) (width 0.2) (layer "F.Cu") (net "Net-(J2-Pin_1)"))
 (segment (start 168.402 68.072) (end 169.227 68.072) (width 0.2) (layer "F.Cu") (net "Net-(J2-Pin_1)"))
 (segment (start 165.1 66.802) (end 165.608 67.31) (width 0.2) (layer "F.Cu") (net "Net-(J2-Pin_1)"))
 (segment (start 165.608 67.31) (end 167.64 67.31) (width 0.2) (layer "F.Cu") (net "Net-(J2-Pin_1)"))
 (segment (start 166.116 62.484) (end 166.116 65.278) (width 0.2) (layer "F.Cu") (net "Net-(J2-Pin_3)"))
 (segment (start 167.132 61.468) (end 166.116 62.484) (width 0.2) (layer "F.Cu") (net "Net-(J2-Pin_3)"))
 (segment (start 166.116 65.278) (end 166.37 65.532) (width 0.2) (layer "F.Cu") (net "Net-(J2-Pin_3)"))
 (segment (start 166.37 65.532) (end 169.227 65.532) (width 0.2) (layer "F.Cu") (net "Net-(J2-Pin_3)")))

